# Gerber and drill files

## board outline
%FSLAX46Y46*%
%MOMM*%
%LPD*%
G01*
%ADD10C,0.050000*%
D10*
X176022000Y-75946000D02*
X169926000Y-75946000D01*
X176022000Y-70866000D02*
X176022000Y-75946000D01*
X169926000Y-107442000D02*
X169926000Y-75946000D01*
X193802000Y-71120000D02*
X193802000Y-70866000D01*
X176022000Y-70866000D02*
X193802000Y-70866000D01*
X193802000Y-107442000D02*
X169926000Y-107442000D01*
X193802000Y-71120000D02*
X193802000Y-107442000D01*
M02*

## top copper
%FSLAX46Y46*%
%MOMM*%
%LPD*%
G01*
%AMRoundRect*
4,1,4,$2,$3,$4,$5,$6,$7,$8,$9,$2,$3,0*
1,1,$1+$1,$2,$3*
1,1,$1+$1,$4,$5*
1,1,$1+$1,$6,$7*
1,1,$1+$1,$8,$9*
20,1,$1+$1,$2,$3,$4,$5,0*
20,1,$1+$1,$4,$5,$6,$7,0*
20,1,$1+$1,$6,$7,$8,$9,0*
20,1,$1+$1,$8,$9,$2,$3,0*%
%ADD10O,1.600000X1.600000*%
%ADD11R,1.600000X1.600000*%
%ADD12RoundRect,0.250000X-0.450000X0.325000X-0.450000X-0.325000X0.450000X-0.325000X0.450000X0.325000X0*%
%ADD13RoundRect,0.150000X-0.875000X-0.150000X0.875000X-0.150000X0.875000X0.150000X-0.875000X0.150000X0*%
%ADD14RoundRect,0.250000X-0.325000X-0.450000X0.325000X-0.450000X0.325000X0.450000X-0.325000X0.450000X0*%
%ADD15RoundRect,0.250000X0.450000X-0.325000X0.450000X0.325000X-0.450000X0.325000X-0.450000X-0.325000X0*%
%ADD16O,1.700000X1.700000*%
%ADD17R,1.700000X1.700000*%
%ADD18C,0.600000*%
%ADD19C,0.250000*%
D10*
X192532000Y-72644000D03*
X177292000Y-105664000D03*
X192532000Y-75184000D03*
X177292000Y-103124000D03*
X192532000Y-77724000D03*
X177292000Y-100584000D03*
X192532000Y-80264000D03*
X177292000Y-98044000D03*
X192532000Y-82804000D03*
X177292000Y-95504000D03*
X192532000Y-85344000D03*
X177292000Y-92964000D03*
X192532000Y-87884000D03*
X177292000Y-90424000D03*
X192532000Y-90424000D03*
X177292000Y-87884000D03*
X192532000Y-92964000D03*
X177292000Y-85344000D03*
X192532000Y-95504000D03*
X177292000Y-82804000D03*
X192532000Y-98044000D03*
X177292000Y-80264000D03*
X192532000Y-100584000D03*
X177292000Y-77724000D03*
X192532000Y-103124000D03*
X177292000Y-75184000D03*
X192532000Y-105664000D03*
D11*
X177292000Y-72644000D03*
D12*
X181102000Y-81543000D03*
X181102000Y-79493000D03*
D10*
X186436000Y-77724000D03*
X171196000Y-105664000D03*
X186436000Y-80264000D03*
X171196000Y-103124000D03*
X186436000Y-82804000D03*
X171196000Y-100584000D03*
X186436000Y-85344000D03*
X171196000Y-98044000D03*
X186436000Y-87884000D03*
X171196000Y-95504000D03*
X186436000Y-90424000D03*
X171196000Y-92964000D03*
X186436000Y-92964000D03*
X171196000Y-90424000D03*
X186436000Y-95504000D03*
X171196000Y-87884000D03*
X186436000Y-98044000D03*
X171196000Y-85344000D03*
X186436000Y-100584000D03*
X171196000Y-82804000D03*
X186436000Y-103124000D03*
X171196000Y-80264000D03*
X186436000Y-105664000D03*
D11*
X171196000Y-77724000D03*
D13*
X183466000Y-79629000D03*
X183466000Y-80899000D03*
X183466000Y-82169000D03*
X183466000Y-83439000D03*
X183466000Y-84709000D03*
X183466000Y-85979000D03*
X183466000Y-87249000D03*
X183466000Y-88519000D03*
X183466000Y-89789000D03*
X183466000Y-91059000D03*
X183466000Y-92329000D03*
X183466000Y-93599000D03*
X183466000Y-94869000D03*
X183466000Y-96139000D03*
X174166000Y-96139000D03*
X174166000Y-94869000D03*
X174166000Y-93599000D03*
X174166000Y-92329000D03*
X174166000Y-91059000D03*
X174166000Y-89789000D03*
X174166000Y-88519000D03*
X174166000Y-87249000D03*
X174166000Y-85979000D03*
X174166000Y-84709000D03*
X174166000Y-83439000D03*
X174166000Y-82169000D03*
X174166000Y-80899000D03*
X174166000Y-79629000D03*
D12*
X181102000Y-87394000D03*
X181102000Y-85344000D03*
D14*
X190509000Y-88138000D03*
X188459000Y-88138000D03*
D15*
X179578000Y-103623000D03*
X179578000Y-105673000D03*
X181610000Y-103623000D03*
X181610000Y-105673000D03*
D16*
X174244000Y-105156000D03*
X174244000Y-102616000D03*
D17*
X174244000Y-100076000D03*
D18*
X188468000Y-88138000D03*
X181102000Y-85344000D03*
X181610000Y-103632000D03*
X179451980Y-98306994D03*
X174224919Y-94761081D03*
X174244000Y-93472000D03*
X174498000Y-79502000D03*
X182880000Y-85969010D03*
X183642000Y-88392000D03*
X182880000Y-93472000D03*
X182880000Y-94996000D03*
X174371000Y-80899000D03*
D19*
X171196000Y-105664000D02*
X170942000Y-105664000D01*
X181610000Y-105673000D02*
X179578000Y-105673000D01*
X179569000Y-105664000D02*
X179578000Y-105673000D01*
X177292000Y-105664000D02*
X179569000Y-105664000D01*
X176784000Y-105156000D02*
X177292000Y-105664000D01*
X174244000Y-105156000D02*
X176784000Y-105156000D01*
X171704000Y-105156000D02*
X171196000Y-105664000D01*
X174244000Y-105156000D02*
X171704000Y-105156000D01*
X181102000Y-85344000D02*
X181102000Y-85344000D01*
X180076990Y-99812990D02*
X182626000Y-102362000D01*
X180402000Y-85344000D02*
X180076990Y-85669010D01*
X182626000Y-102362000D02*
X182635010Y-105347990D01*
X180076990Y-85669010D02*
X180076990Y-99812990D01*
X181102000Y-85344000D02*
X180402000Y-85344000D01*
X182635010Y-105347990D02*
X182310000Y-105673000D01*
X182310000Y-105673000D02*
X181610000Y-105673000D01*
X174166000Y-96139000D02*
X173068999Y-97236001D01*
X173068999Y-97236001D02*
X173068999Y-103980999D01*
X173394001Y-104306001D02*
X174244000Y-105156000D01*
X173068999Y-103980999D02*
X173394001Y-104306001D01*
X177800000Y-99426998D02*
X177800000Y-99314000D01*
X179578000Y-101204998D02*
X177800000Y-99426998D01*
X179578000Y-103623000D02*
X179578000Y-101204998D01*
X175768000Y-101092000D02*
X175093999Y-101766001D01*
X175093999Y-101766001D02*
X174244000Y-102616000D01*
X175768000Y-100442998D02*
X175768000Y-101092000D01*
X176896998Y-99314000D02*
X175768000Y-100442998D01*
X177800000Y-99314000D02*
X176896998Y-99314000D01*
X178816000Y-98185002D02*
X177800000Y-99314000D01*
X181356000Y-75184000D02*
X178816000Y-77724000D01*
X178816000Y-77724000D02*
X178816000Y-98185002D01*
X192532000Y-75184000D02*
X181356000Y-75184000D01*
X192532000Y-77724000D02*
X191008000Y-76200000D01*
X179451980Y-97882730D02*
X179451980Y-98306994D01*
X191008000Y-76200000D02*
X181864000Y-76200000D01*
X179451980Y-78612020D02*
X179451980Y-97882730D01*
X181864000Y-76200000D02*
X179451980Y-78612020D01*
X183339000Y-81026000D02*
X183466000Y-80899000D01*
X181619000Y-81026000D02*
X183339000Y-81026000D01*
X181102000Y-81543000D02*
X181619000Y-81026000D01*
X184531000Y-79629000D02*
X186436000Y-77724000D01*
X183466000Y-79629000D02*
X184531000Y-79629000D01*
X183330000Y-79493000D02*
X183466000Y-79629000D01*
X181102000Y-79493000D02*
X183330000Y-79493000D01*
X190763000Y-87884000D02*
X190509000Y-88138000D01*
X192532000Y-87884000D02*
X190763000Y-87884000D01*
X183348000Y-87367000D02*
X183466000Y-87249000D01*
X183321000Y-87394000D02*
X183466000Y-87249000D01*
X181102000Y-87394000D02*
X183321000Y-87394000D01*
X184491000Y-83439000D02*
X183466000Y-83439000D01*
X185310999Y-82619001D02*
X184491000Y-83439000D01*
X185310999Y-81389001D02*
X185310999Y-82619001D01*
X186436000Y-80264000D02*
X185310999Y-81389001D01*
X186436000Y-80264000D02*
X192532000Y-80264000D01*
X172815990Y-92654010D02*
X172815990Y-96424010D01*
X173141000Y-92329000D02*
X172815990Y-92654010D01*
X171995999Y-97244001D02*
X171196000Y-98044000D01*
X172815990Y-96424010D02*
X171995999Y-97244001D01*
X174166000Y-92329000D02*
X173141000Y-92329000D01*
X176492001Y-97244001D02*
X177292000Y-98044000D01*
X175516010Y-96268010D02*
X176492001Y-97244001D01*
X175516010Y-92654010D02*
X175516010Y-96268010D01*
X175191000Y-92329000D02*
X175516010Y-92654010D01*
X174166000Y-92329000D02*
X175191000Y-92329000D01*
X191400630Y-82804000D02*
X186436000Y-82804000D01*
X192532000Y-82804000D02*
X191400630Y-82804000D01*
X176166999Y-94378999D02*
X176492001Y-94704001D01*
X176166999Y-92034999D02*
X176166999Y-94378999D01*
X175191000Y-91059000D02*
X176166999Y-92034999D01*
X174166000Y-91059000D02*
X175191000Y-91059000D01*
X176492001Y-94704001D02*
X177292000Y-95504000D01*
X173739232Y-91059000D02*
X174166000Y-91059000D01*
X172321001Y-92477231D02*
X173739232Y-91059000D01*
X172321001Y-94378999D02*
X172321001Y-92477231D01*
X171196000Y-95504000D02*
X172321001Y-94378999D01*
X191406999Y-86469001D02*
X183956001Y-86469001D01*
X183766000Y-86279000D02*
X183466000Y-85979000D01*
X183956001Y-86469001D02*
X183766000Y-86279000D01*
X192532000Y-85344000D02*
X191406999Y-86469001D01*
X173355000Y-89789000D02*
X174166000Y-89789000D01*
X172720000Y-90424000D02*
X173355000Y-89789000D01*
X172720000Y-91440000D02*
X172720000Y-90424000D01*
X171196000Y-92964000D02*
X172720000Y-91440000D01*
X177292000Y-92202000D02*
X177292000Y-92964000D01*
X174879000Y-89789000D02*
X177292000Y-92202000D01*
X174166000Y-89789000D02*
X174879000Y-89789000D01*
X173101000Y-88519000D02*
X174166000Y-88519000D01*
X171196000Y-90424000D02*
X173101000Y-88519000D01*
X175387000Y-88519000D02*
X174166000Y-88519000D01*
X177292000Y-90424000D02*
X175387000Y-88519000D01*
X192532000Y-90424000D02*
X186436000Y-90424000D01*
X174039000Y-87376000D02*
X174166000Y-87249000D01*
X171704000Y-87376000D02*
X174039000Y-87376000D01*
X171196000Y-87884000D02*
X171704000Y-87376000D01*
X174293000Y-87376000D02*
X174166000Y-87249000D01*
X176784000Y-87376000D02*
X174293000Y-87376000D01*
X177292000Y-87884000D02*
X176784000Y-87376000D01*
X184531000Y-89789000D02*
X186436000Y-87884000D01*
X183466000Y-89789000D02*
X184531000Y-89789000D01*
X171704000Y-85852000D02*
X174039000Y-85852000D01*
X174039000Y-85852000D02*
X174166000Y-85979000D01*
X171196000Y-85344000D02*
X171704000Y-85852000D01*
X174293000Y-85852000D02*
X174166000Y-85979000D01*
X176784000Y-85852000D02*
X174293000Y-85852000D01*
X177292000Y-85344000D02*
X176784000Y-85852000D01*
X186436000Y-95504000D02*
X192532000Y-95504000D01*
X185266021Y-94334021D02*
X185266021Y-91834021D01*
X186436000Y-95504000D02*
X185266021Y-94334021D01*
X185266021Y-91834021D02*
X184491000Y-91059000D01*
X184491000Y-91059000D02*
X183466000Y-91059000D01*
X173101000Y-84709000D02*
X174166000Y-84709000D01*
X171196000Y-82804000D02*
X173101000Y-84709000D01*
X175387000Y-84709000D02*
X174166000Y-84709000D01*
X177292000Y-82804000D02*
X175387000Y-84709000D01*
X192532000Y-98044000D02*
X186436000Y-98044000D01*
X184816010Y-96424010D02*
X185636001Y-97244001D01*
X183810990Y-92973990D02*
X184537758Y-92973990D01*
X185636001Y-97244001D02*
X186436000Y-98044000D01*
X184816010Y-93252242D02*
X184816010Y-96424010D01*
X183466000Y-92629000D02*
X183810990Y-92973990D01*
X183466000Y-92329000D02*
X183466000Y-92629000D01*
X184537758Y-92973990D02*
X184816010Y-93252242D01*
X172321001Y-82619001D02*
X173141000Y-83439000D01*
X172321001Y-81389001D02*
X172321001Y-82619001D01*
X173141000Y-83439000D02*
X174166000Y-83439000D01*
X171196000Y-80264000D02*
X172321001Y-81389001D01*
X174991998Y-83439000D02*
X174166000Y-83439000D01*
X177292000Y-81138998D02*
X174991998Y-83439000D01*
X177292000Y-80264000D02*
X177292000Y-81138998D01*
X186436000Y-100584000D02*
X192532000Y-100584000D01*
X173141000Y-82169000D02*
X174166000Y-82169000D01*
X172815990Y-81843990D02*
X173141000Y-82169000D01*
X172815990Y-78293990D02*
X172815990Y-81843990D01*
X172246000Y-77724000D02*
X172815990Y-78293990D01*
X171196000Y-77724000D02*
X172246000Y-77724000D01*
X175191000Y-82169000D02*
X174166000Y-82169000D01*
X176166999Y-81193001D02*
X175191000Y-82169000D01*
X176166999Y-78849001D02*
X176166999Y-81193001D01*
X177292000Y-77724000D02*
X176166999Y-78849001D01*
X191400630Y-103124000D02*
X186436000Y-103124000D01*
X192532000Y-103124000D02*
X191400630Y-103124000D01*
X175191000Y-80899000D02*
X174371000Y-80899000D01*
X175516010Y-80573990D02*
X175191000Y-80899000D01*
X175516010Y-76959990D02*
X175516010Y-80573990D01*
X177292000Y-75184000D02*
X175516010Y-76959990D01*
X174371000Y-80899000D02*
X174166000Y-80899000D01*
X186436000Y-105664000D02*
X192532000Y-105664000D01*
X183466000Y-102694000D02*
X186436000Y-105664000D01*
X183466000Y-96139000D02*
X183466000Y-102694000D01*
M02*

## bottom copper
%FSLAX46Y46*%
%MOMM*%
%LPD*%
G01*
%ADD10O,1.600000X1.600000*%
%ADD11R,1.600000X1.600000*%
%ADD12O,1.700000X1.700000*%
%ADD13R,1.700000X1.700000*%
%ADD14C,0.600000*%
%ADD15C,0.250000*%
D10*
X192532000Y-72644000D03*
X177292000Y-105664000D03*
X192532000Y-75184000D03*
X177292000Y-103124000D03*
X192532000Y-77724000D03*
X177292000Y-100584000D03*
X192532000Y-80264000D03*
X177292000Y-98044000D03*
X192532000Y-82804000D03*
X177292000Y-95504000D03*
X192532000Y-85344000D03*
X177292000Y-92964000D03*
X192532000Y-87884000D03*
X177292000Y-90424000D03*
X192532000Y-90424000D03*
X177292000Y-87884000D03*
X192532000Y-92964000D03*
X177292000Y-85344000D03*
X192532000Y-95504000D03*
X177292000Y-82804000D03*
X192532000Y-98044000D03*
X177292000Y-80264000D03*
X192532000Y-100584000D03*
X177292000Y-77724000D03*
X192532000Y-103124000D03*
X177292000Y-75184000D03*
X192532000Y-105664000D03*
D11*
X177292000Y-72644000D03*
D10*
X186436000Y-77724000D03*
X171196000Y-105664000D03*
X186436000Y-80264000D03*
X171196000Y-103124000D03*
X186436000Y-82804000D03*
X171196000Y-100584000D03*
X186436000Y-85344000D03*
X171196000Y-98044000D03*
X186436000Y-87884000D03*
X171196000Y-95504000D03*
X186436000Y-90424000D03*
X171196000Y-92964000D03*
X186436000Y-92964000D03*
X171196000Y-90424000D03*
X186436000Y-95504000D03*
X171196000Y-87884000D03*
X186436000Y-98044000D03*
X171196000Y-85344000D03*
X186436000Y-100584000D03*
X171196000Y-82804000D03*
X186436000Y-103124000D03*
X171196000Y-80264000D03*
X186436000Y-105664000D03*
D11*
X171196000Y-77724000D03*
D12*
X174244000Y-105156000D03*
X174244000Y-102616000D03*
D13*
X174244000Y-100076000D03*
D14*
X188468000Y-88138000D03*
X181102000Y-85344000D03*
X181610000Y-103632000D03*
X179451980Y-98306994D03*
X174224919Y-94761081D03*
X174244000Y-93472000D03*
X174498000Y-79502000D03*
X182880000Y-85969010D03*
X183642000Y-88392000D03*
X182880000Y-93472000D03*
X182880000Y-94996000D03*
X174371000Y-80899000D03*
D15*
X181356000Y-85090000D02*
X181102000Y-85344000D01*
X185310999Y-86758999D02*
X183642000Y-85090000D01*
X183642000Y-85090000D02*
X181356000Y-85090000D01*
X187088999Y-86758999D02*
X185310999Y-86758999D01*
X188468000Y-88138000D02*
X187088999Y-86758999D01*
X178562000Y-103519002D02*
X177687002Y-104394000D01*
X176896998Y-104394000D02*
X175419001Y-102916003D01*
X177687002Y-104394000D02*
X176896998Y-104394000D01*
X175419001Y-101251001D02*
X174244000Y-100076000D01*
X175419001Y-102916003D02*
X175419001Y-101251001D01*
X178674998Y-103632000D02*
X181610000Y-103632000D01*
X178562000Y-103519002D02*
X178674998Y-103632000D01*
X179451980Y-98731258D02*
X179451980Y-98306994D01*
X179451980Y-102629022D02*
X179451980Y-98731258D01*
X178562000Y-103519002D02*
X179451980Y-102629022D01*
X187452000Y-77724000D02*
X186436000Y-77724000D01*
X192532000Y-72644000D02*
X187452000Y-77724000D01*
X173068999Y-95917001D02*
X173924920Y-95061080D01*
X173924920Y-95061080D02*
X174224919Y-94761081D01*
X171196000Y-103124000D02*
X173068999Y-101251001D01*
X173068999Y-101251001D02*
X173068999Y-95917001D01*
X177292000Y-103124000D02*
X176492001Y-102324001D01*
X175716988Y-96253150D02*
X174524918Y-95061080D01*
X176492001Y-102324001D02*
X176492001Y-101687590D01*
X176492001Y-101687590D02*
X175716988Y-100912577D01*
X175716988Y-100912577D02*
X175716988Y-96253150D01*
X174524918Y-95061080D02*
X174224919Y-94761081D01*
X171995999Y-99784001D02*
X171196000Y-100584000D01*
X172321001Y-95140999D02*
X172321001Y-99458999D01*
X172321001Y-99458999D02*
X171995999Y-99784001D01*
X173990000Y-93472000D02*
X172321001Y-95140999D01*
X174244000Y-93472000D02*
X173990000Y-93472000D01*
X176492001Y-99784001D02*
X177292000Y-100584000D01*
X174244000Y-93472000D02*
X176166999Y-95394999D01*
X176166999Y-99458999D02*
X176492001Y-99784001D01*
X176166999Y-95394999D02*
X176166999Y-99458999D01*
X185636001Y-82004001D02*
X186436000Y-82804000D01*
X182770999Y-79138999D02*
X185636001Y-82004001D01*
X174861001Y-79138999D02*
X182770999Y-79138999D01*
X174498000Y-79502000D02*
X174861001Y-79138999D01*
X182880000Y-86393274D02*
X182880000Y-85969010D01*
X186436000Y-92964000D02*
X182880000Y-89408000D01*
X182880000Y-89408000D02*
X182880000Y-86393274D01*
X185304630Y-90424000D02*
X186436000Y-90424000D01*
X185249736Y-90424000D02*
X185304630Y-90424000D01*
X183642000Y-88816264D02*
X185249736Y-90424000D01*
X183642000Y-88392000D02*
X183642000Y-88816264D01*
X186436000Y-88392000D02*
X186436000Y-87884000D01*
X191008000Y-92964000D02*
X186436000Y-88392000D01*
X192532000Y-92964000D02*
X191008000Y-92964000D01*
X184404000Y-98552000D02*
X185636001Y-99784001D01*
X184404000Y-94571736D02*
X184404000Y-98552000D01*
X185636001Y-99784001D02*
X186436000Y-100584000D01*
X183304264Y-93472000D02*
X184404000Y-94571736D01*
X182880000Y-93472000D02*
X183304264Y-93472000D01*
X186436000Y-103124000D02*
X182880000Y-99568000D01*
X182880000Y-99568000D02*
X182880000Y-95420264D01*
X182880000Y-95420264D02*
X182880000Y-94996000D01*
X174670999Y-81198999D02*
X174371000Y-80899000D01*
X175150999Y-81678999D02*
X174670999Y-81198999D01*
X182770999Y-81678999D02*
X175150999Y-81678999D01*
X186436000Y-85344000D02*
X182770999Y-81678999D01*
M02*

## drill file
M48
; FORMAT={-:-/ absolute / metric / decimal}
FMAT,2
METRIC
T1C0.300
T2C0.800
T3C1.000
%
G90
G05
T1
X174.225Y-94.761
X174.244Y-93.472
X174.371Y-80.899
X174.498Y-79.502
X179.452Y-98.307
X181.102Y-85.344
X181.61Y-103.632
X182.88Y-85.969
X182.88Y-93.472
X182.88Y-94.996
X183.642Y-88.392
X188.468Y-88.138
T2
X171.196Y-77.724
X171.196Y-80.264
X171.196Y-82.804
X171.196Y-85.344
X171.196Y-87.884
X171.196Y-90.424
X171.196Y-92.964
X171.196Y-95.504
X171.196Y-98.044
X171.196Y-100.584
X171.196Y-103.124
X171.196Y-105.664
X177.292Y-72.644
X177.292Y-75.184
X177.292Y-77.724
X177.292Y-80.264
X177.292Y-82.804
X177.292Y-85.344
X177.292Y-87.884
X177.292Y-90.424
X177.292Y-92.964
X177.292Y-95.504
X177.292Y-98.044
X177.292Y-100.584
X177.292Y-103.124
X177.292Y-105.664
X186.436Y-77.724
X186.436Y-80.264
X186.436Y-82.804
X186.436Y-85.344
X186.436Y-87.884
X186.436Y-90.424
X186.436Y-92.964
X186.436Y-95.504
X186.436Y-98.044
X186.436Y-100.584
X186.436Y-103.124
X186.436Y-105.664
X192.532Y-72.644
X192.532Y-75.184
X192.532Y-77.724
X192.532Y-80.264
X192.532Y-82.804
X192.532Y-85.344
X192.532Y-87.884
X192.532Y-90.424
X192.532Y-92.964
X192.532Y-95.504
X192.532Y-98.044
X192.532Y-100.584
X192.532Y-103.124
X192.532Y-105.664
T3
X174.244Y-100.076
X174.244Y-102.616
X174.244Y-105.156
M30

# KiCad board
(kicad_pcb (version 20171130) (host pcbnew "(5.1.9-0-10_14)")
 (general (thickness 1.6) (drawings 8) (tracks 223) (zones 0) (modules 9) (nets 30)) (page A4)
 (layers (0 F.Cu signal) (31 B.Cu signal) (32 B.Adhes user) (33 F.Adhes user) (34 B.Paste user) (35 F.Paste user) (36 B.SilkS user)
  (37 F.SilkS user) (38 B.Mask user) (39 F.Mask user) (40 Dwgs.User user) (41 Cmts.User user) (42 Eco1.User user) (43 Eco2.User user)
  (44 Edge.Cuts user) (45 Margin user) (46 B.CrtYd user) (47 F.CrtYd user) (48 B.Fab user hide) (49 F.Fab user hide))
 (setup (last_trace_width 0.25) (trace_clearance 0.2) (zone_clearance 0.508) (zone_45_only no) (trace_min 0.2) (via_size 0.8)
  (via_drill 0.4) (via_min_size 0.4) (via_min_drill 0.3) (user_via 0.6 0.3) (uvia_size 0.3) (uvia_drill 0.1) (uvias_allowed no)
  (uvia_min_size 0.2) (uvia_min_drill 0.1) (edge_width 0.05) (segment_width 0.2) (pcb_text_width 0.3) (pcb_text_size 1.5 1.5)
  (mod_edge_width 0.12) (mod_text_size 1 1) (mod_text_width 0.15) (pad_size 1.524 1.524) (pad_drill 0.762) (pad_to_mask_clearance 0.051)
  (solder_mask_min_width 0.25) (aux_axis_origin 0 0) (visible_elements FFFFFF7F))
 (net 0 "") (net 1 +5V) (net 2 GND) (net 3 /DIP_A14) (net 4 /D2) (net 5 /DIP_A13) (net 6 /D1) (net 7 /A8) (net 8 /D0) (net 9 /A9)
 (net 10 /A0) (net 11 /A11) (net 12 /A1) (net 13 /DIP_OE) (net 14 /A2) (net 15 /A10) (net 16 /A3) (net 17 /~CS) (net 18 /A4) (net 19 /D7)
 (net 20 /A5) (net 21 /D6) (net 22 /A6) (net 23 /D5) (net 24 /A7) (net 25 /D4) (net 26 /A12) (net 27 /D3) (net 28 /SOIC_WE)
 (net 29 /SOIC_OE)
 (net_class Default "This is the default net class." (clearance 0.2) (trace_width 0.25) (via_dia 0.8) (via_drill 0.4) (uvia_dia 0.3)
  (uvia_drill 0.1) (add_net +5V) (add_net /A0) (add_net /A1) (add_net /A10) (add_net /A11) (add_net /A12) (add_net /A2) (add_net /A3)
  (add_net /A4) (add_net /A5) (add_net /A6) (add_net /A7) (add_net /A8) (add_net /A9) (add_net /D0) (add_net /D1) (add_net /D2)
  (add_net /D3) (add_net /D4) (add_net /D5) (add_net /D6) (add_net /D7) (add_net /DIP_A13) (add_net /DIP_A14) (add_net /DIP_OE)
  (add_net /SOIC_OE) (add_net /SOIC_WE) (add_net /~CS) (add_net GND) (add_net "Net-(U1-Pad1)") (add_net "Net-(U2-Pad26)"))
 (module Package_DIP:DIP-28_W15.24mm (layer F.Cu) (at 177.292 72.644)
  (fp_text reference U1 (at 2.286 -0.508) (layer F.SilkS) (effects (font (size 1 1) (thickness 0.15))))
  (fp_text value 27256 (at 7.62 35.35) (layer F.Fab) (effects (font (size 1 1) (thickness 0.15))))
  (pad 28 thru_hole oval (at 15.24 0) (size 1.6 1.6) (drill 0.8) (layers *.Cu *.Mask) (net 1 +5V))
  (pad 14 thru_hole oval (at 0 33.02) (size 1.6 1.6) (drill 0.8) (layers *.Cu *.Mask) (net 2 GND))
  (pad 27 thru_hole oval (at 15.24 2.54) (size 1.6 1.6) (drill 0.8) (layers *.Cu *.Mask) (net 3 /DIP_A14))
  (pad 13 thru_hole oval (at 0 30.48) (size 1.6 1.6) (drill 0.8) (layers *.Cu *.Mask) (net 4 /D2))
  (pad 26 thru_hole oval (at 15.24 5.08) (size 1.6 1.6) (drill 0.8) (layers *.Cu *.Mask) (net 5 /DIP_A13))
  (pad 12 thru_hole oval (at 0 27.94) (size 1.6 1.6) (drill 0.8) (layers *.Cu *.Mask) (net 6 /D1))
  (pad 25 thru_hole oval (at 15.24 7.62) (size 1.6 1.6) (drill 0.8) (layers *.Cu *.Mask) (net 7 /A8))
  (pad 11 thru_hole oval (at 0 25.4) (size 1.6 1.6) (drill 0.8) (layers *.Cu *.Mask) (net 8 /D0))
  (pad 24 thru_hole oval (at 15.24 10.16) (size 1.6 1.6) (drill 0.8) (layers *.Cu *.Mask) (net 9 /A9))
  (pad 10 thru_hole oval (at 0 22.86) (size 1.6 1.6) (drill 0.8) (layers *.Cu *.Mask) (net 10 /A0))
  (pad 23 thru_hole oval (at 15.24 12.7) (size 1.6 1.6) (drill 0.8) (layers *.Cu *.Mask) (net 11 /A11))
  (pad 9 thru_hole oval (at 0 20.32) (size 1.6 1.6) (drill 0.8) (layers *.Cu *.Mask) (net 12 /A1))
  (pad 22 thru_hole oval (at 15.24 15.24) (size 1.6 1.6) (drill 0.8) (layers *.Cu *.Mask) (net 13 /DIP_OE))
  (pad 8 thru_hole oval (at 0 17.78) (size 1.6 1.6) (drill 0.8) (layers *.Cu *.Mask) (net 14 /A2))
  (pad 21 thru_hole oval (at 15.24 17.78) (size 1.6 1.6) (drill 0.8) (layers *.Cu *.Mask) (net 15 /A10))
  (pad 7 thru_hole oval (at 0 15.24) (size 1.6 1.6) (drill 0.8) (layers *.Cu *.Mask) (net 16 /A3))
  (pad 20 thru_hole oval (at 15.24 20.32) (size 1.6 1.6) (drill 0.8) (layers *.Cu *.Mask) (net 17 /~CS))
  (pad 6 thru_hole oval (at 0 12.7) (size 1.6 1.6) (drill 0.8) (layers *.Cu *.Mask) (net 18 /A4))
  (pad 19 thru_hole oval (at 15.24 22.86) (size 1.6 1.6) (drill 0.8) (layers *.Cu *.Mask) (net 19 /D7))
  (pad 5 thru_hole oval (at 0 10.16) (size 1.6 1.6) (drill 0.8) (layers *.Cu *.Mask) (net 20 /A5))
  (pad 18 thru_hole oval (at 15.24 25.4) (size 1.6 1.6) (drill 0.8) (layers *.Cu *.Mask) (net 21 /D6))
  (pad 4 thru_hole oval (at 0 7.62) (size 1.6 1.6) (drill 0.8) (layers *.Cu *.Mask) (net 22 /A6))
  (pad 17 thru_hole oval (at 15.24 27.94) (size 1.6 1.6) (drill 0.8) (layers *.Cu *.Mask) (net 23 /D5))
  (pad 3 thru_hole oval (at 0 5.08) (size 1.6 1.6) (drill 0.8) (layers *.Cu *.Mask) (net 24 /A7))
  (pad 16 thru_hole oval (at 15.24 30.48) (size 1.6 1.6) (drill 0.8) (layers *.Cu *.Mask) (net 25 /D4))
  (pad 2 thru_hole oval (at 0 2.54) (size 1.6 1.6) (drill 0.8) (layers *.Cu *.Mask) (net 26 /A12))
  (pad 15 thru_hole oval (at 15.24 33.02) (size 1.6 1.6) (drill 0.8) (layers *.Cu *.Mask) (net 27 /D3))
  (pad 1 thru_hole rect (at 0 0) (size 1.6 1.6) (drill 0.8) (layers *.Cu *.Mask)))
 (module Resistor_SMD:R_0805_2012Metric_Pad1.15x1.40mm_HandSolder (layer F.Cu) (at 181.102 80.518 270)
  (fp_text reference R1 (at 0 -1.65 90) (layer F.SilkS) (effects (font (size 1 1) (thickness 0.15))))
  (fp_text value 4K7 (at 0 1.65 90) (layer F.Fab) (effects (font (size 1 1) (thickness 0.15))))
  (pad 2 smd roundrect (at 1.025 0 270) (size 1.15 1.4) (layers F.Cu F.Paste F.Mask) (roundrect_rratio 0.217391) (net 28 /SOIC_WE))
  (pad 1 smd roundrect (at -1.025 0 270) (size 1.15 1.4) (layers F.Cu F.Paste F.Mask) (roundrect_rratio 0.217391) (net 1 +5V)))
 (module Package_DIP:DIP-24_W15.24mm (layer F.Cu) (at 171.196 77.724)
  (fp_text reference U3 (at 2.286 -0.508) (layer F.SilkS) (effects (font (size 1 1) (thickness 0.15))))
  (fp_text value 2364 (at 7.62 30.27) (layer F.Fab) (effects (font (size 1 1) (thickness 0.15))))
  (pad 24 thru_hole oval (at 15.24 0) (size 1.6 1.6) (drill 0.8) (layers *.Cu *.Mask) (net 1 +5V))
  (pad 12 thru_hole oval (at 0 27.94) (size 1.6 1.6) (drill 0.8) (layers *.Cu *.Mask) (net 2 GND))
  (pad 23 thru_hole oval (at 15.24 2.54) (size 1.6 1.6) (drill 0.8) (layers *.Cu *.Mask) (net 7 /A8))
  (pad 11 thru_hole oval (at 0 25.4) (size 1.6 1.6) (drill 0.8) (layers *.Cu *.Mask) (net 4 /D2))
  (pad 22 thru_hole oval (at 15.24 5.08) (size 1.6 1.6) (drill 0.8) (layers *.Cu *.Mask) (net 9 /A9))
  (pad 10 thru_hole oval (at 0 22.86) (size 1.6 1.6) (drill 0.8) (layers *.Cu *.Mask) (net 6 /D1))
  (pad 21 thru_hole oval (at 15.24 7.62) (size 1.6 1.6) (drill 0.8) (layers *.Cu *.Mask) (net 26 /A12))
  (pad 9 thru_hole oval (at 0 20.32) (size 1.6 1.6) (drill 0.8) (layers *.Cu *.Mask) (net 8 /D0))
  (pad 20 thru_hole oval (at 15.24 10.16) (size 1.6 1.6) (drill 0.8) (layers *.Cu *.Mask) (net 17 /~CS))
  (pad 8 thru_hole oval (at 0 17.78) (size 1.6 1.6) (drill 0.8) (layers *.Cu *.Mask) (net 10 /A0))
  (pad 19 thru_hole oval (at 15.24 12.7) (size 1.6 1.6) (drill 0.8) (layers *.Cu *.Mask) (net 15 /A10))
  (pad 7 thru_hole oval (at 0 15.24) (size 1.6 1.6) (drill 0.8) (layers *.Cu *.Mask) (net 12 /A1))
  (pad 18 thru_hole oval (at 15.24 15.24) (size 1.6 1.6) (drill 0.8) (layers *.Cu *.Mask) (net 11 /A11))
  (pad 6 thru_hole oval (at 0 12.7) (size 1.6 1.6) (drill 0.8) (layers *.Cu *.Mask) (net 14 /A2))
  (pad 17 thru_hole oval (at 15.24 17.78) (size 1.6 1.6) (drill 0.8) (layers *.Cu *.Mask) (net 19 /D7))
  (pad 5 thru_hole oval (at 0 10.16) (size 1.6 1.6) (drill 0.8) (layers *.Cu *.Mask) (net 16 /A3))
  (pad 16 thru_hole oval (at 15.24 20.32) (size 1.6 1.6) (drill 0.8) (layers *.Cu *.Mask) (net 21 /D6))
  (pad 4 thru_hole oval (at 0 7.62) (size 1.6 1.6) (drill 0.8) (layers *.Cu *.Mask) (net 18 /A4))
  (pad 15 thru_hole oval (at 15.24 22.86) (size 1.6 1.6) (drill 0.8) (layers *.Cu *.Mask) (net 23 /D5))
  (pad 3 thru_hole oval (at 0 5.08) (size 1.6 1.6) (drill 0.8) (layers *.Cu *.Mask) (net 20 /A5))
  (pad 14 thru_hole oval (at 15.24 25.4) (size 1.6 1.6) (drill 0.8) (layers *.Cu *.Mask) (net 25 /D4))
  (pad 2 thru_hole oval (at 0 2.54) (size 1.6 1.6) (drill 0.8) (layers *.Cu *.Mask) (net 22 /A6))
  (pad 13 thru_hole oval (at 15.24 27.94) (size 1.6 1.6) (drill 0.8) (layers *.Cu *.Mask) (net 27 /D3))
  (pad 1 thru_hole rect (at 0 0) (size 1.6 1.6) (drill 0.8) (layers *.Cu *.Mask) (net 24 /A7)))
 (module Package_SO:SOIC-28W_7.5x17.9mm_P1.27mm (layer F.Cu) (at 178.816 87.884)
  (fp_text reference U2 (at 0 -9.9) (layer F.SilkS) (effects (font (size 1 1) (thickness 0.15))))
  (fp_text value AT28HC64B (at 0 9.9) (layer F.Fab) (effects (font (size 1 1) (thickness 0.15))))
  (pad 28 smd roundrect (at 4.65 -8.255) (size 2.05 0.6) (layers F.Cu F.Paste F.Mask) (roundrect_rratio 0.25) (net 1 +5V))
  (pad 27 smd roundrect (at 4.65 -6.985) (size 2.05 0.6) (layers F.Cu F.Paste F.Mask) (roundrect_rratio 0.25) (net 28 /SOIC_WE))
  (pad 26 smd roundrect (at 4.65 -5.715) (size 2.05 0.6) (layers F.Cu F.Paste F.Mask) (roundrect_rratio 0.25))
  (pad 25 smd roundrect (at 4.65 -4.445) (size 2.05 0.6) (layers F.Cu F.Paste F.Mask) (roundrect_rratio 0.25) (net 7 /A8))
  (pad 24 smd roundrect (at 4.65 -3.175) (size 2.05 0.6) (layers F.Cu F.Paste F.Mask) (roundrect_rratio 0.25))
  (pad 23 smd roundrect (at 4.65 -1.905) (size 2.05 0.6) (layers F.Cu F.Paste F.Mask) (roundrect_rratio 0.25) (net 11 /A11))
  (pad 22 smd roundrect (at 4.65 -0.635) (size 2.05 0.6) (layers F.Cu F.Paste F.Mask) (roundrect_rratio 0.25) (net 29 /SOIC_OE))
  (pad 21 smd roundrect (at 4.65 0.635) (size 2.05 0.6) (layers F.Cu F.Paste F.Mask) (roundrect_rratio 0.25) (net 15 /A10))
  (pad 20 smd roundrect (at 4.65 1.905) (size 2.05 0.6) (layers F.Cu F.Paste F.Mask) (roundrect_rratio 0.25) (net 17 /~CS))
  (pad 19 smd roundrect (at 4.65 3.175) (size 2.05 0.6) (layers F.Cu F.Paste F.Mask) (roundrect_rratio 0.25) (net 19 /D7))
  (pad 18 smd roundrect (at 4.65 4.445) (size 2.05 0.6) (layers F.Cu F.Paste F.Mask) (roundrect_rratio 0.25) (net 21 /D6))
  (pad 17 smd roundrect (at 4.65 5.715) (size 2.05 0.6) (layers F.Cu F.Paste F.Mask) (roundrect_rratio 0.25) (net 23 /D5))
  (pad 16 smd roundrect (at 4.65 6.985) (size 2.05 0.6) (layers F.Cu F.Paste F.Mask) (roundrect_rratio 0.25) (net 25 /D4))
  (pad 15 smd roundrect (at 4.65 8.255) (size 2.05 0.6) (layers F.Cu F.Paste F.Mask) (roundrect_rratio 0.25) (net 27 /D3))
  (pad 14 smd roundrect (at -4.65 8.255) (size 2.05 0.6) (layers F.Cu F.Paste F.Mask) (roundrect_rratio 0.25) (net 2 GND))
  (pad 13 smd roundrect (at -4.65 6.985) (size 2.05 0.6) (layers F.Cu F.Paste F.Mask) (roundrect_rratio 0.25) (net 4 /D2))
  (pad 12 smd roundrect (at -4.65 5.715) (size 2.05 0.6) (layers F.Cu F.Paste F.Mask) (roundrect_rratio 0.25) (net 6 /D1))
  (pad 11 smd roundrect (at -4.65 4.445) (size 2.05 0.6) (layers F.Cu F.Paste F.Mask) (roundrect_rratio 0.25) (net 8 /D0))
  (pad 10 smd roundrect (at -4.65 3.175) (size 2.05 0.6) (layers F.Cu F.Paste F.Mask) (roundrect_rratio 0.25) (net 10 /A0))
  (pad 9 smd roundrect (at -4.65 1.905) (size 2.05 0.6) (layers F.Cu F.Paste F.Mask) (roundrect_rratio 0.25) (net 12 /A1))
  (pad 8 smd roundrect (at -4.65 0.635) (size 2.05 0.6) (layers F.Cu F.Paste F.Mask) (roundrect_rratio 0.25) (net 14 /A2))
  (pad 7 smd roundrect (at -4.65 -0.635) (size 2.05 0.6) (layers F.Cu F.Paste F.Mask) (roundrect_rratio 0.25) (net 16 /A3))
  (pad 6 smd roundrect (at -4.65 -1.905) (size 2.05 0.6) (layers F.Cu F.Paste F.Mask) (roundrect_rratio 0.25) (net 18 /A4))
  (pad 5 smd roundrect (at -4.65 -3.175) (size 2.05 0.6) (layers F.Cu F.Paste F.Mask) (roundrect_rratio 0.25) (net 20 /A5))
  (pad 4 smd roundrect (at -4.65 -4.445) (size 2.05 0.6) (layers F.Cu F.Paste F.Mask) (roundrect_rratio 0.25) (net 22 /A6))
  (pad 3 smd roundrect (at -4.65 -5.715) (size 2.05 0.6) (layers F.Cu F.Paste F.Mask) (roundrect_rratio 0.25) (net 24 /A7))
  (pad 2 smd roundrect (at -4.65 -6.985) (size 2.05 0.6) (layers F.Cu F.Paste F.Mask) (roundrect_rratio 0.25) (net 26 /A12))
  (pad 1 smd roundrect (at -4.65 -8.255) (size 2.05 0.6) (layers F.Cu F.Paste F.Mask) (roundrect_rratio 0.25) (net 9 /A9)))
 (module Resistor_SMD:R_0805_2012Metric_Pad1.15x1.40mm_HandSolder (layer F.Cu) (at 181.102 86.369 270)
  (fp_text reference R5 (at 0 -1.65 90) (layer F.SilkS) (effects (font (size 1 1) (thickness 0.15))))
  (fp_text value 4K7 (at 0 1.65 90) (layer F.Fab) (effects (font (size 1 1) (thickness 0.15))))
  (pad 2 smd roundrect (at 1.025 0 270) (size 1.15 1.4) (layers F.Cu F.Paste F.Mask) (roundrect_rratio 0.217391) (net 29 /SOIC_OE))
  (pad 1 smd roundrect (at -1.025 0 270) (size 1.15 1.4) (layers F.Cu F.Paste F.Mask) (roundrect_rratio 0.217391) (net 2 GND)))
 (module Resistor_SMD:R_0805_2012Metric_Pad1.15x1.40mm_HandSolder (layer F.Cu) (at 189.484 88.138)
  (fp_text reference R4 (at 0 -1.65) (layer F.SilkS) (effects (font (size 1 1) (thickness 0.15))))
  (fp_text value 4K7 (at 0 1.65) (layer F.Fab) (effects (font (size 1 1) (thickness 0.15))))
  (pad 2 smd roundrect (at 1.025 0) (size 1.15 1.4) (layers F.Cu F.Paste F.Mask) (roundrect_rratio 0.217391) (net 13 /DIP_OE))
  (pad 1 smd roundrect (at -1.025 0) (size 1.15 1.4) (layers F.Cu F.Paste F.Mask) (roundrect_rratio 0.217391) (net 2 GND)))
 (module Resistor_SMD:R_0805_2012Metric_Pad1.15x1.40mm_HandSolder (layer F.Cu) (at 179.578 104.648 90)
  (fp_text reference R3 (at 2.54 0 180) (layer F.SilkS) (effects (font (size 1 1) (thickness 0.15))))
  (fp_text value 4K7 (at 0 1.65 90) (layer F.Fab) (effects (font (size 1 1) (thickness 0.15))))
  (pad 2 smd roundrect (at 1.025 0 90) (size 1.15 1.4) (layers F.Cu F.Paste F.Mask) (roundrect_rratio 0.217391) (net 3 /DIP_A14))
  (pad 1 smd roundrect (at -1.025 0 90) (size 1.15 1.4) (layers F.Cu F.Paste F.Mask) (roundrect_rratio 0.217391) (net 2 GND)))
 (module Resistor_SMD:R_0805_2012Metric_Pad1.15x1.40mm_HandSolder (layer F.Cu) (at 181.61 104.648 90)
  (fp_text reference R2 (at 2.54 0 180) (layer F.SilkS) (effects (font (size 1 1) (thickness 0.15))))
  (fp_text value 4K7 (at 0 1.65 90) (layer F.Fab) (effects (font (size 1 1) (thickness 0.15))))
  (pad 2 smd roundrect (at 1.025 0 90) (size 1.15 1.4) (layers F.Cu F.Paste F.Mask) (roundrect_rratio 0.217391) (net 5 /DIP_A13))
  (pad 1 smd roundrect (at -1.025 0 90) (size 1.15 1.4) (layers F.Cu F.Paste F.Mask) (roundrect_rratio 0.217391) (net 2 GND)))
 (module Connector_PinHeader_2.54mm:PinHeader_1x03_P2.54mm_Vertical (layer F.Cu) (at 174.244 100.076)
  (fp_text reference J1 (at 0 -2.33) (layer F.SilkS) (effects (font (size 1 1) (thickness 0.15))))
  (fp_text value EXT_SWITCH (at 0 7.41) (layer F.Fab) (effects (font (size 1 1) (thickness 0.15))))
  (pad 3 thru_hole oval (at 0 5.08) (size 1.7 1.7) (drill 1) (layers *.Cu *.Mask) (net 2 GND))
  (pad 2 thru_hole oval (at 0 2.54) (size 1.7 1.7) (drill 1) (layers *.Cu *.Mask) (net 3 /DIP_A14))
  (pad 1 thru_hole rect (at 0 0) (size 1.7 1.7) (drill 1) (layers *.Cu *.Mask) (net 5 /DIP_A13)))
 (gr_line (start 176.022 75.946) (end 169.926 75.946) (layer Edge.Cuts) (width 0.05))
 (gr_line (start 176.022 70.866) (end 176.022 75.946) (layer Edge.Cuts) (width 0.05))
 (gr_line (start 169.926 107.442) (end 169.926 75.946) (layer Edge.Cuts) (width 0.05))
 (gr_line (start 193.802 71.12) (end 193.802 70.866) (layer Edge.Cuts) (width 0.05))
 (gr_line (start 176.022 70.866) (end 193.802 70.866) (layer Edge.Cuts) (width 0.05))
 (gr_line (start 193.802 107.442) (end 169.926 107.442) (layer Edge.Cuts) (width 0.05))
 (gr_line (start 193.802 71.12) (end 193.802 107.442) (layer Edge.Cuts) (width 0.05))
 (via (at 188.468 88.138) (size 0.6) (drill 0.3) (layers F.Cu B.Cu) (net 2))
 (segment (start 171.196 105.664) (end 170.942 105.664) (width 0.25) (layer F.Cu) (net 2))
 (segment (start 181.61 105.673) (end 179.578 105.673) (width 0.25) (layer F.Cu) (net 2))
 (segment (start 179.569 105.664) (end 179.578 105.673) (width 0.25) (layer F.Cu) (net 2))
 (segment (start 177.292 105.664) (end 179.569 105.664) (width 0.25) (layer F.Cu) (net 2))
 (segment (start 176.784 105.156) (end 177.292 105.664) (width 0.25) (layer F.Cu) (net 2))
 (segment (start 174.244 105.156) (end 176.784 105.156) (width 0.25) (layer F.Cu) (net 2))
 (segment (start 171.704 105.156) (end 171.196 105.664) (width 0.25) (layer F.Cu) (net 2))
 (segment (start 174.244 105.156) (end 171.704 105.156) (width 0.25) (layer F.Cu) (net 2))
 (segment (start 181.102 85.344) (end 181.102 85.344) (width 0.25) (layer F.Cu) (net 2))
 (via (at 181.102 85.344) (size 0.6) (drill 0.3) (layers F.Cu B.Cu) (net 2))
 (segment (start 181.356 85.09) (end 181.102 85.344) (width 0.25) (layer B.Cu) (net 2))
 (segment (start 185.310999 86.758999) (end 183.642 85.09) (width 0.25) (layer B.Cu) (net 2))
 (segment (start 183.642 85.09) (end 181.356 85.09) (width 0.25) (layer B.Cu) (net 2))
 (segment (start 187.088999 86.758999) (end 185.310999 86.758999) (width 0.25) (layer B.Cu) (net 2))
 (segment (start 188.468 88.138) (end 187.088999 86.758999) (width 0.25) (layer B.Cu) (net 2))
 (segment (start 180.07699 99.81299) (end 182.626 102.362) (width 0.25) (layer F.Cu) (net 2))
 (segment (start 180.402 85.344) (end 180.07699 85.66901) (width 0.25) (layer F.Cu) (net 2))
 (segment (start 182.626 102.362) (end 182.63501 105.34799) (width 0.25) (layer F.Cu) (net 2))
 (segment (start 180.07699 85.66901) (end 180.07699 99.81299) (width 0.25) (layer F.Cu) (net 2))
 (segment (start 181.102 85.344) (end 180.402 85.344) (width 0.25) (layer F.Cu) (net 2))
 (segment (start 182.63501 105.34799) (end 182.31 105.673) (width 0.25) (layer F.Cu) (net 2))
 (segment (start 182.31 105.673) (end 181.61 105.673) (width 0.25) (layer F.Cu) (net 2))
 (segment (start 174.166 96.139) (end 173.068999 97.236001) (width 0.25) (layer F.Cu) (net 2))
 (segment (start 173.068999 97.236001) (end 173.068999 103.980999) (width 0.25) (layer F.Cu) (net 2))
 (segment (start 173.394001 104.306001) (end 174.244 105.156) (width 0.25) (layer F.Cu) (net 2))
 (segment (start 173.068999 103.980999) (end 173.394001 104.306001) (width 0.25) (layer F.Cu) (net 2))
 (segment (start 177.8 99.426998) (end 177.8 99.314) (width 0.25) (layer F.Cu) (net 3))
 (segment (start 179.578 101.204998) (end 177.8 99.426998) (width 0.25) (layer F.Cu) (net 3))
 (segment (start 179.578 103.623) (end 179.578 101.204998) (width 0.25) (layer F.Cu) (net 3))
 (segment (start 175.768 101.092) (end 175.093999 101.766001) (width 0.25) (layer F.Cu) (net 3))
 (segment (start 175.093999 101.766001) (end 174.244 102.616) (width 0.25) (layer F.Cu) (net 3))
 (segment (start 175.768 100.442998) (end 175.768 101.092) (width 0.25) (layer F.Cu) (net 3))
 (segment (start 176.896998 99.314) (end 175.768 100.442998) (width 0.25) (layer F.Cu) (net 3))
 (segment (start 177.8 99.314) (end 176.896998 99.314) (width 0.25) (layer F.Cu) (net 3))
 (segment (start 178.816 98.185002) (end 177.8 99.314) (width 0.25) (layer F.Cu) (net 3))
 (segment (start 181.356 75.184) (end 178.816 77.724) (width 0.25) (layer F.Cu) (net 3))
 (segment (start 178.816 77.724) (end 178.816 98.185002) (width 0.25) (layer F.Cu) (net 3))
 (segment (start 192.532 75.184) (end 181.356 75.184) (width 0.25) (layer F.Cu) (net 3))
 (via (at 181.61 103.632) (size 0.6) (drill 0.3) (layers F.Cu B.Cu) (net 5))
 (segment (start 178.562 103.519002) (end 177.687002 104.394) (width 0.25) (layer B.Cu) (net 5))
 (segment (start 176.896998 104.394) (end 175.419001 102.916003) (width 0.25) (layer B.Cu) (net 5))
 (segment (start 177.687002 104.394) (end 176.896998 104.394) (width 0.25) (layer B.Cu) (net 5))
 (segment (start 175.419001 101.251001) (end 174.244 100.076) (width 0.25) (layer B.Cu) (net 5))
 (segment (start 175.419001 102.916003) (end 175.419001 101.251001) (width 0.25) (layer B.Cu) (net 5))
 (segment (start 178.674998 103.632) (end 181.61 103.632) (width 0.25) (layer B.Cu) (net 5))
 (segment (start 178.562 103.519002) (end 178.674998 103.632) (width 0.25) (layer B.Cu) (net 5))
 (segment (start 179.45198 98.731258) (end 179.45198 98.306994) (width 0.25) (layer B.Cu) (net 5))
 (segment (start 179.45198 102.629022) (end 179.45198 98.731258) (width 0.25) (layer B.Cu) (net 5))
 (via (at 179.45198 98.306994) (size 0.6) (drill 0.3) (layers F.Cu B.Cu) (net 5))
 (segment (start 178.562 103.519002) (end 179.45198 102.629022) (width 0.25) (layer B.Cu) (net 5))
 (segment (start 192.532 77.724) (end 191.008 76.2) (width 0.25) (layer F.Cu) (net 5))
 (segment (start 179.45198 97.88273) (end 179.45198 98.306994) (width 0.25) (layer F.Cu) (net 5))
 (segment (start 191.008 76.2) (end 181.864 76.2) (width 0.25) (layer F.Cu) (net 5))
 (segment (start 179.45198 78.61202) (end 179.45198 97.88273) (width 0.25) (layer F.Cu) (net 5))
 (segment (start 181.864 76.2) (end 179.45198 78.61202) (width 0.25) (layer F.Cu) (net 5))
 (segment (start 183.339 81.026) (end 183.466 80.899) (width 0.25) (layer F.Cu) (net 28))
 (segment (start 181.619 81.026) (end 183.339 81.026) (width 0.25) (layer F.Cu) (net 28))
 (segment (start 181.102 81.543) (end 181.619 81.026) (width 0.25) (layer F.Cu) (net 28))
 (segment (start 187.452 77.724) (end 186.436 77.724) (width 0.25) (layer B.Cu) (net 1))
 (segment (start 192.532 72.644) (end 187.452 77.724) (width 0.25) (layer B.Cu) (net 1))
 (segment (start 184.531 79.629) (end 186.436 77.724) (width 0.25) (layer F.Cu) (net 1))
 (segment (start 183.466 79.629) (end 184.531 79.629) (width 0.25) (layer F.Cu) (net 1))
 (segment (start 183.33 79.493) (end 183.466 79.629) (width 0.25) (layer F.Cu) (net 1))
 (segment (start 181.102 79.493) (end 183.33 79.493) (width 0.25) (layer F.Cu) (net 1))
 (segment (start 190.763 87.884) (end 190.509 88.138) (width 0.25) (layer F.Cu) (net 13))
 (segment (start 192.532 87.884) (end 190.763 87.884) (width 0.25) (layer F.Cu) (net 13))
 (segment (start 183.348 87.367) (end 183.466 87.249) (width 0.25) (layer F.Cu) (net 29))
 (segment (start 183.321 87.394) (end 183.466 87.249) (width 0.25) (layer F.Cu) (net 29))
 (segment (start 181.102 87.394) (end 183.321 87.394) (width 0.25) (layer F.Cu) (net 29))
 (segment (start 173.068999 95.917001) (end 173.92492 95.06108) (width 0.25) (layer B.Cu) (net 4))
 (segment (start 173.92492 95.06108) (end 174.224919 94.761081) (width 0.25) (layer B.Cu) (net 4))
 (segment (start 171.196 103.124) (end 173.068999 101.251001) (width 0.25) (layer B.Cu) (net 4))
 (via (at 174.224919 94.761081) (size 0.6) (drill 0.3) (layers F.Cu B.Cu) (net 4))
 (segment (start 173.068999 101.251001) (end 173.068999 95.917001) (width 0.25) (layer B.Cu) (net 4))
 (segment (start 177.292 103.124) (end 176.492001 102.324001) (width 0.25) (layer B.Cu) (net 4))
 (segment (start 175.716988 96.25315) (end 174.524918 95.06108) (width 0.25) (layer B.Cu) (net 4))
 (segment (start 176.492001 102.324001) (end 176.492001 101.68759) (width 0.25) (layer B.Cu) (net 4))
 (segment (start 176.492001 101.68759) (end 175.716988 100.912577) (width 0.25) (layer B.Cu) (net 4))
 (segment (start 175.716988 100.912577) (end 175.716988 96.25315) (width 0.25) (layer B.Cu) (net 4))
 (segment (start 174.524918 95.06108) (end 174.224919 94.761081) (width 0.25) (layer B.Cu) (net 4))
 (via (at 174.244 93.472) (size 0.6) (drill 0.3) (layers F.Cu B.Cu) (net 6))
 (segment (start 171.995999 99.784001) (end 171.196 100.584) (width 0.25) (layer B.Cu) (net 6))
 (segment (start 172.321001 95.140999) (end 172.321001 99.458999) (width 0.25) (layer B.Cu) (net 6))
 (segment (start 172.321001 99.458999) (end 171.995999 99.784001) (width 0.25) (layer B.Cu) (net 6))
 (segment (start 173.99 93.472) (end 172.321001 95.140999) (width 0.25) (layer B.Cu) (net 6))
 (segment (start 174.244 93.472) (end 173.99 93.472) (width 0.25) (layer B.Cu) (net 6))
 (segment (start 176.492001 99.784001) (end 177.292 100.584) (width 0.25) (layer B.Cu) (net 6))
 (segment (start 174.244 93.472) (end 176.166999 95.394999) (width 0.25) (layer B.Cu) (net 6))
 (segment (start 176.166999 99.458999) (end 176.492001 99.784001) (width 0.25) (layer B.Cu) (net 6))
 (segment (start 176.166999 95.394999) (end 176.166999 99.458999) (width 0.25) (layer B.Cu) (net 6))
 (segment (start 184.491 83.439) (end 183.466 83.439) (width 0.25) (layer F.Cu) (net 7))
 (segment (start 185.310999 82.619001) (end 184.491 83.439) (width 0.25) (layer F.Cu) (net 7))
 (segment (start 185.310999 81.389001) (end 185.310999 82.619001) (width 0.25) (layer F.Cu) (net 7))
 (segment (start 186.436 80.264) (end 185.310999 81.389001) (width 0.25) (layer F.Cu) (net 7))
 (segment (start 186.436 80.264) (end 192.532 80.264) (width 0.25) (layer F.Cu) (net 7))
 (segment (start 172.81599 92.65401) (end 172.81599 96.42401) (width 0.25) (layer F.Cu) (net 8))
 (segment (start 173.141 92.329) (end 172.81599 92.65401) (width 0.25) (layer F.Cu) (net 8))
 (segment (start 171.995999 97.244001) (end 171.196 98.044) (width 0.25) (layer F.Cu) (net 8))
 (segment (start 172.81599 96.42401) (end 171.995999 97.244001) (width 0.25) (layer F.Cu) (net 8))
 (segment (start 174.166 92.329) (end 173.141 92.329) (width 0.25) (layer F.Cu) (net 8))
 (segment (start 176.492001 97.244001) (end 177.292 98.044) (width 0.25) (layer F.Cu) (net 8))
 (segment (start 175.51601 96.26801) (end 176.492001 97.244001) (width 0.25) (layer F.Cu) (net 8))
 (segment (start 175.51601 92.65401) (end 175.51601 96.26801) (width 0.25) (layer F.Cu) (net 8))
 (segment (start 175.191 92.329) (end 175.51601 92.65401) (width 0.25) (layer F.Cu) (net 8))
 (segment (start 174.166 92.329) (end 175.191 92.329) (width 0.25) (layer F.Cu) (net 8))
 (via (at 174.498 79.502) (size 0.6) (drill 0.3) (layers F.Cu B.Cu) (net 9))
 (segment (start 191.40063 82.804) (end 186.436 82.804) (width 0.25) (layer F.Cu) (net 9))
 (segment (start 192.532 82.804) (end 191.40063 82.804) (width 0.25) (layer F.Cu) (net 9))
 (segment (start 185.636001 82.004001) (end 186.436 82.804) (width 0.25) (layer B.Cu) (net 9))
 (segment (start 182.770999 79.138999) (end 185.636001 82.004001) (width 0.25) (layer B.Cu) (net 9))
 (segment (start 174.861001 79.138999) (end 182.770999 79.138999) (width 0.25) (layer B.Cu) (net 9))
 (segment (start 174.498 79.502) (end 174.861001 79.138999) (width 0.25) (layer B.Cu) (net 9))
 (segment (start 176.166999 94.378999) (end 176.492001 94.704001) (width 0.25) (layer F.Cu) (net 10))
 (segment (start 176.166999 92.034999) (end 176.166999 94.378999) (width 0.25) (layer F.Cu) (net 10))
 (segment (start 175.191 91.059) (end 176.166999 92.034999) (width 0.25) (layer F.Cu) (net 10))
 (segment (start 174.166 91.059) (end 175.191 91.059) (width 0.25) (layer F.Cu) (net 10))
 (segment (start 176.492001 94.704001) (end 177.292 95.504) (width 0.25) (layer F.Cu) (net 10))
 (segment (start 173.739232 91.059) (end 174.166 91.059) (width 0.25) (layer F.Cu) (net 10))
 (segment (start 172.321001 92.477231) (end 173.739232 91.059) (width 0.25) (layer F.Cu) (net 10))
 (segment (start 172.321001 94.378999) (end 172.321001 92.477231) (width 0.25) (layer F.Cu) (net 10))
 (segment (start 171.196 95.504) (end 172.321001 94.378999) (width 0.25) (layer F.Cu) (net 10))
 (segment (start 191.406999 86.469001) (end 183.956001 86.469001) (width 0.25) (layer F.Cu) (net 11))
 (segment (start 183.766 86.279) (end 183.466 85.979) (width 0.25) (layer F.Cu) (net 11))
 (segment (start 183.956001 86.469001) (end 183.766 86.279) (width 0.25) (layer F.Cu) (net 11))
 (segment (start 192.532 85.344) (end 191.406999 86.469001) (width 0.25) (layer F.Cu) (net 11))
 (via (at 182.88 85.96901) (size 0.6) (drill 0.3) (layers F.Cu B.Cu) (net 11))
 (segment (start 182.88 86.393274) (end 182.88 85.96901) (width 0.25) (layer B.Cu) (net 11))
 (segment (start 186.436 92.964) (end 182.88 89.408) (width 0.25) (layer B.Cu) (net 11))
 (segment (start 182.88 89.408) (end 182.88 86.393274) (width 0.25) (layer B.Cu) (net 11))
 (segment (start 173.355 89.789) (end 174.166 89.789) (width 0.25) (layer F.Cu) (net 12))
 (segment (start 172.72 90.424) (end 173.355 89.789) (width 0.25) (layer F.Cu) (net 12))
 (segment (start 172.72 91.44) (end 172.72 90.424) (width 0.25) (layer F.Cu) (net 12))
 (segment (start 171.196 92.964) (end 172.72 91.44) (width 0.25) (layer F.Cu) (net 12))
 (segment (start 177.292 92.202) (end 177.292 92.964) (width 0.25) (layer F.Cu) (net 12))
 (segment (start 174.879 89.789) (end 177.292 92.202) (width 0.25) (layer F.Cu) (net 12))
 (segment (start 174.166 89.789) (end 174.879 89.789) (width 0.25) (layer F.Cu) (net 12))
 (segment (start 173.101 88.519) (end 174.166 88.519) (width 0.25) (layer F.Cu) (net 14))
 (segment (start 171.196 90.424) (end 173.101 88.519) (width 0.25) (layer F.Cu) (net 14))
 (segment (start 175.387 88.519) (end 174.166 88.519) (width 0.25) (layer F.Cu) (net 14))
 (segment (start 177.292 90.424) (end 175.387 88.519) (width 0.25) (layer F.Cu) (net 14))
 (via (at 183.642 88.392) (size 0.6) (drill 0.3) (layers F.Cu B.Cu) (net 15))
 (segment (start 192.532 90.424) (end 186.436 90.424) (width 0.25) (layer F.Cu) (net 15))
 (segment (start 185.30463 90.424) (end 186.436 90.424) (width 0.25) (layer B.Cu) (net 15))
 (segment (start 185.249736 90.424) (end 185.30463 90.424) (width 0.25) (layer B.Cu) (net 15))
 (segment (start 183.642 88.816264) (end 185.249736 90.424) (width 0.25) (layer B.Cu) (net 15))
 (segment (start 183.642 88.392) (end 183.642 88.816264) (width 0.25) (layer B.Cu) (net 15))
 (segment (start 174.039 87.376) (end 174.166 87.249) (width 0.25) (layer F.Cu) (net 16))
 (segment (start 171.704 87.376) (end 174.039 87.376) (width 0.25) (layer F.Cu) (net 16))
 (segment (start 171.196 87.884) (end 171.704 87.376) (width 0.25) (layer F.Cu) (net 16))
 (segment (start 174.293 87.376) (end 174.166 87.249) (width 0.25) (layer F.Cu) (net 16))
 (segment (start 176.784 87.376) (end 174.293 87.376) (width 0.25) (layer F.Cu) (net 16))
 (segment (start 177.292 87.884) (end 176.784 87.376) (width 0.25) (layer F.Cu) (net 16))
 (segment (start 184.531 89.789) (end 186.436 87.884) (width 0.25) (layer F.Cu) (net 17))
 (segment (start 183.466 89.789) (end 184.531 89.789) (width 0.25) (layer F.Cu) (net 17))
 (segment (start 186.436 88.392) (end 186.436 87.884) (width 0.25) (layer B.Cu) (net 17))
 (segment (start 191.008 92.964) (end 186.436 88.392) (width 0.25) (layer B.Cu) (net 17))
 (segment (start 192.532 92.964) (end 191.008 92.964) (width 0.25) (layer B.Cu) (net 17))
 (segment (start 171.704 85.852) (end 174.039 85.852) (width 0.25) (layer F.Cu) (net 18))
 (segment (start 174.039 85.852) (end 174.166 85.979) (width 0.25) (layer F.Cu) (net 18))
 (segment (start 171.196 85.344) (end 171.704 85.852) (width 0.25) (layer F.Cu) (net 18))
 (segment (start 174.293 85.852) (end 174.166 85.979) (width 0.25) (layer F.Cu) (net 18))
 (segment (start 176.784 85.852) (end 174.293 85.852) (width 0.25) (layer F.Cu) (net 18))
 (segment (start 177.292 85.344) (end 176.784 85.852) (width 0.25) (layer F.Cu) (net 18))
 (segment (start 186.436 95.504) (end 192.532 95.504) (width 0.25) (layer F.Cu) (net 19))
 (segment (start 185.266021 94.334021) (end 185.266021 91.834021) (width 0.25) (layer F.Cu) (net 19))
 (segment (start 186.436 95.504) (end 185.266021 94.334021) (width 0.25) (layer F.Cu) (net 19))
 (segment (start 185.266021 91.834021) (end 184.491 91.059) (width 0.25) (layer F.Cu) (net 19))
 (segment (start 184.491 91.059) (end 183.466 91.059) (width 0.25) (layer F.Cu) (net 19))
 (segment (start 173.101 84.709) (end 174.166 84.709) (width 0.25) (layer F.Cu) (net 20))
 (segment (start 171.196 82.804) (end 173.101 84.709) (width 0.25) (layer F.Cu) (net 20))
 (segment (start 175.387 84.709) (end 174.166 84.709) (width 0.25) (layer F.Cu) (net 20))
 (segment (start 177.292 82.804) (end 175.387 84.709) (width 0.25) (layer F.Cu) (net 20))
 (segment (start 192.532 98.044) (end 186.436 98.044) (width 0.25) (layer F.Cu) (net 21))
 (segment (start 184.81601 96.42401) (end 185.636001 97.244001) (width 0.25) (layer F.Cu) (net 21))
 (segment (start 183.81099 92.97399) (end 184.537758 92.97399) (width 0.25) (layer F.Cu) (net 21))
 (segment (start 185.636001 97.244001) (end 186.436 98.044) (width 0.25) (layer F.Cu) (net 21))
 (segment (start 184.81601 93.252242) (end 184.81601 96.42401) (width 0.25) (layer F.Cu) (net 21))
 (segment (start 183.466 92.629) (end 183.81099 92.97399) (width 0.25) (layer F.Cu) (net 21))
 (segment (start 183.466 92.329) (end 183.466 92.629) (width 0.25) (layer F.Cu) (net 21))
 (segment (start 184.537758 92.97399) (end 184.81601 93.252242) (width 0.25) (layer F.Cu) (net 21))
 (segment (start 172.321001 82.619001) (end 173.141 83.439) (width 0.25) (layer F.Cu) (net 22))
 (segment (start 172.321001 81.389001) (end 172.321001 82.619001) (width 0.25) (layer F.Cu) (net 22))
 (segment (start 173.141 83.439) (end 174.166 83.439) (width 0.25) (layer F.Cu) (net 22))
 (segment (start 171.196 80.264) (end 172.321001 81.389001) (width 0.25) (layer F.Cu) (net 22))
 (segment (start 174.991998 83.439) (end 174.166 83.439) (width 0.25) (layer F.Cu) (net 22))
 (segment (start 177.292 81.138998) (end 174.991998 83.439) (width 0.25) (layer F.Cu) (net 22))
 (segment (start 177.292 80.264) (end 177.292 81.138998) (width 0.25) (layer F.Cu) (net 22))
 (via (at 182.88 93.472) (size 0.6) (drill 0.3) (layers F.Cu B.Cu) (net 23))
 (segment (start 186.436 100.584) (end 192.532 100.584) (width 0.25) (layer F.Cu) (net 23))
 (segment (start 184.404 98.552) (end 185.636001 99.784001) (width 0.25) (layer B.Cu) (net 23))
 (segment (start 184.404 94.571736) (end 184.404 98.552) (width 0.25) (layer B.Cu) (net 23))
 (segment (start 185.636001 99.784001) (end 186.436 100.584) (width 0.25) (layer B.Cu) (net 23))
 (segment (start 183.304264 93.472) (end 184.404 94.571736) (width 0.25) (layer B.Cu) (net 23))
 (segment (start 182.88 93.472) (end 183.304264 93.472) (width 0.25) (layer B.Cu) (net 23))
 (segment (start 173.141 82.169) (end 174.166 82.169) (width 0.25) (layer F.Cu) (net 24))
 (segment (start 172.81599 81.84399) (end 173.141 82.169) (width 0.25) (layer F.Cu) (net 24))
 (segment (start 172.81599 78.29399) (end 172.81599 81.84399) (width 0.25) (layer F.Cu) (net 24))
 (segment (start 172.246 77.724) (end 172.81599 78.29399) (width 0.25) (layer F.Cu) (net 24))
 (segment (start 171.196 77.724) (end 172.246 77.724) (width 0.25) (layer F.Cu) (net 24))
 (segment (start 175.191 82.169) (end 174.166 82.169) (width 0.25) (layer F.Cu) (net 24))
 (segment (start 176.166999 81.193001) (end 175.191 82.169) (width 0.25) (layer F.Cu) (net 24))
 (segment (start 176.166999 78.849001) (end 176.166999 81.193001) (width 0.25) (layer F.Cu) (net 24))
 (segment (start 177.292 77.724) (end 176.166999 78.849001) (width 0.25) (layer F.Cu) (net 24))
 (segment (start 191.40063 103.124) (end 186.436 103.124) (width 0.25) (layer F.Cu) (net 25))
 (segment (start 192.532 103.124) (end 191.40063 103.124) (width 0.25) (layer F.Cu) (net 25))
 (via (at 182.88 94.996) (size 0.6) (drill 0.3) (layers F.Cu B.Cu) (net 25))
 (segment (start 186.436 103.124) (end 182.88 99.568) (width 0.25) (layer B.Cu) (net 25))
 (segment (start 182.88 99.568) (end 182.88 95.420264) (width 0.25) (layer B.Cu) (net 25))
 (segment (start 182.88 95.420264) (end 182.88 94.996) (width 0.25) (layer B.Cu) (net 25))
 (segment (start 175.191 80.899) (end 174.371 80.899) (width 0.25) (layer F.Cu) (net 26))
 (segment (start 175.51601 80.57399) (end 175.191 80.899) (width 0.25) (layer F.Cu) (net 26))
 (segment (start 175.51601 76.95999) (end 175.51601 80.57399) (width 0.25) (layer F.Cu) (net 26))
 (segment (start 177.292 75.184) (end 175.51601 76.95999) (width 0.25) (layer F.Cu) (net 26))
 (segment (start 174.371 80.899) (end 174.166 80.899) (width 0.25) (layer F.Cu) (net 26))
 (via (at 174.371 80.899) (size 0.6) (drill 0.3) (layers F.Cu B.Cu) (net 26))
 (segment (start 174.670999 81.198999) (end 174.371 80.899) (width 0.25) (layer B.Cu) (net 26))
 (segment (start 175.150999 81.678999) (end 174.670999 81.198999) (width 0.25) (layer B.Cu) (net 26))
 (segment (start 182.770999 81.678999) (end 175.150999 81.678999) (width 0.25) (layer B.Cu) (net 26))
 (segment (start 186.436 85.344) (end 182.770999 81.678999) (width 0.25) (layer B.Cu) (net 26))
 (segment (start 186.436 105.664) (end 192.532 105.664) (width 0.25) (layer F.Cu) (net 27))
 (segment (start 183.466 102.694) (end 186.436 105.664) (width 0.25) (layer F.Cu) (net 27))
 (segment (start 183.466 96.139) (end 183.466 102.694) (width 0.25) (layer F.Cu) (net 27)))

